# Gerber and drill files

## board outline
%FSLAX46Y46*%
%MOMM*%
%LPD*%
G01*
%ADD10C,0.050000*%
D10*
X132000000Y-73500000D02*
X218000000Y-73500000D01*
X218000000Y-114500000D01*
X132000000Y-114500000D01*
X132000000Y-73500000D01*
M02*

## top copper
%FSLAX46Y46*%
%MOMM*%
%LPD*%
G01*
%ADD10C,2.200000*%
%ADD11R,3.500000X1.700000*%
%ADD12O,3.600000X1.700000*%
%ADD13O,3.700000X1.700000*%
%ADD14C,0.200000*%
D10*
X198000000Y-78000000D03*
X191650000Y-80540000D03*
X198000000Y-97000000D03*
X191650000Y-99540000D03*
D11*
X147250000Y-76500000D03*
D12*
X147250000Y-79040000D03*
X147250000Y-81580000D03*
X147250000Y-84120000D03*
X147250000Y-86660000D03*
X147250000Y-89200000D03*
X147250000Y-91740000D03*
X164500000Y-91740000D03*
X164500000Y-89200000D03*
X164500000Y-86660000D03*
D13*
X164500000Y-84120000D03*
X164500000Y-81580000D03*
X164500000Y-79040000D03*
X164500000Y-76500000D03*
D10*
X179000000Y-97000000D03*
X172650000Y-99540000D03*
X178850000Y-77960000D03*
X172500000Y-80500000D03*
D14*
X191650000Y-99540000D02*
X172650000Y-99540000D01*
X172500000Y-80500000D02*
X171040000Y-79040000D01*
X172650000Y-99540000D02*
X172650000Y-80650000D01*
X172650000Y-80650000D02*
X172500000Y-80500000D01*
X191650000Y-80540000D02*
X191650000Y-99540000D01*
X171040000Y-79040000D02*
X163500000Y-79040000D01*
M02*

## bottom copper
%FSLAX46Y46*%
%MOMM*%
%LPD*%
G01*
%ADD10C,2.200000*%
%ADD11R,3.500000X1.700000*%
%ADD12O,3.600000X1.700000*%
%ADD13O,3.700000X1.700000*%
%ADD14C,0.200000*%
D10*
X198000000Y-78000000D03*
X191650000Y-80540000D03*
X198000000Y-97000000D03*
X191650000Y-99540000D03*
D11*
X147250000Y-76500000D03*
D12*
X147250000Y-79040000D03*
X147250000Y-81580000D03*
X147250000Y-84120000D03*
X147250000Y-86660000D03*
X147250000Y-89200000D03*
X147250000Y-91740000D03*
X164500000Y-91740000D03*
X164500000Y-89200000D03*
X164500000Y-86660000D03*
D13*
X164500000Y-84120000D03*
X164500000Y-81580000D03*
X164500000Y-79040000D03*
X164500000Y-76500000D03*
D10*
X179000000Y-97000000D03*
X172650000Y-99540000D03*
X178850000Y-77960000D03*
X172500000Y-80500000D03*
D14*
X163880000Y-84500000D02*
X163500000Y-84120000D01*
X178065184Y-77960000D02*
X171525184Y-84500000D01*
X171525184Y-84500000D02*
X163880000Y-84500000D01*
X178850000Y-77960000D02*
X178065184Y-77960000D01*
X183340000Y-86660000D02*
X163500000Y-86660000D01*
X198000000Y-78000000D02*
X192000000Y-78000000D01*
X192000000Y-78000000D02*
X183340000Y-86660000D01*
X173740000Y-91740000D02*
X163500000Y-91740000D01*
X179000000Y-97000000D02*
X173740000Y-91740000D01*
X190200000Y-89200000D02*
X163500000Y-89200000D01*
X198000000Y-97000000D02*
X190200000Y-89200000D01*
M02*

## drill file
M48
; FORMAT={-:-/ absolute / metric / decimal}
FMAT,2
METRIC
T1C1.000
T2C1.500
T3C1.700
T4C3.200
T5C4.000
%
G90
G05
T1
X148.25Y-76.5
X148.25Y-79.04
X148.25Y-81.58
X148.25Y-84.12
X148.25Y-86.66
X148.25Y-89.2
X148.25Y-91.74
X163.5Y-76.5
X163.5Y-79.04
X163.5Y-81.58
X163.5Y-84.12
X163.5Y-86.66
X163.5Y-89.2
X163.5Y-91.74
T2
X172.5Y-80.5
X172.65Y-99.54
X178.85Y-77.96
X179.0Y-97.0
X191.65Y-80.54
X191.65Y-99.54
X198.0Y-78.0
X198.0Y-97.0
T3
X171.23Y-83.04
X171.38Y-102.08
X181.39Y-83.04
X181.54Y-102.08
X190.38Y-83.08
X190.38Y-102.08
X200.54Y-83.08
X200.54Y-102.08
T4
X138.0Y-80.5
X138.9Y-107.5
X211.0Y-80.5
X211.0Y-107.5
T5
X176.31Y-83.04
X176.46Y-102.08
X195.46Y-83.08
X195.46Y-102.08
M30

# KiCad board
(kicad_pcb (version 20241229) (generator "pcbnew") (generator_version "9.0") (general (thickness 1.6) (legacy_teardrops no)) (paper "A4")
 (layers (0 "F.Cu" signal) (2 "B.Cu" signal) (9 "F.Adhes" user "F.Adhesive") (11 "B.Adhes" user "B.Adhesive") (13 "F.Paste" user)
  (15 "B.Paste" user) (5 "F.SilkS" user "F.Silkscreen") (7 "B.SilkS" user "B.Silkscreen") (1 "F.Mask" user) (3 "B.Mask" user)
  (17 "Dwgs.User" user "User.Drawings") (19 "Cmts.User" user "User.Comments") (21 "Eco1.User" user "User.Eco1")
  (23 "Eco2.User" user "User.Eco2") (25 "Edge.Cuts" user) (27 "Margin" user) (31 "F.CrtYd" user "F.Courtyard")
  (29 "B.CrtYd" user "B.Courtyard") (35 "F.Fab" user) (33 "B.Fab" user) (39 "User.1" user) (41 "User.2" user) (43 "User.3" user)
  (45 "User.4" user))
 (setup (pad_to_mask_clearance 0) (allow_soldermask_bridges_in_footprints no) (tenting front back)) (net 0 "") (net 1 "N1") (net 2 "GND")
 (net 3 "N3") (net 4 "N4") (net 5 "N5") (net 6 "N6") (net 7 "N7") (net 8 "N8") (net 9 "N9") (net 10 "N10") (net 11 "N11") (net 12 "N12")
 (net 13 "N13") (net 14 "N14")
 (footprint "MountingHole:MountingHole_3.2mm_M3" (layer "F.Cu") (at 138.9 107.5)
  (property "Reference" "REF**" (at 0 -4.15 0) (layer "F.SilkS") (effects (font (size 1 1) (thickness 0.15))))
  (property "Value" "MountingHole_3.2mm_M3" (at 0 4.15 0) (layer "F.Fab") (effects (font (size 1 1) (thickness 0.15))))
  (pad "" np_thru_hole circle (at 0 0) (size 3.2 3.2) (drill 3.2) (layers "*.Cu" "*.Mask")))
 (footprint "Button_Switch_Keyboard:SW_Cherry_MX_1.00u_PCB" (layer "F.Cu") (at 198 78)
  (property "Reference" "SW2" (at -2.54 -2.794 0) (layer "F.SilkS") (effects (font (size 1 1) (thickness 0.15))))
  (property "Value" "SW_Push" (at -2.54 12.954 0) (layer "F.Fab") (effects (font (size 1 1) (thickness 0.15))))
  (pad "" np_thru_hole circle (at -7.62 5.08) (size 1.7 1.7) (drill 1.7) (layers "*.Cu" "*.Mask"))
  (pad "" np_thru_hole circle (at -2.54 5.08) (size 4 4) (drill 4) (layers "*.Cu" "*.Mask"))
  (pad "" np_thru_hole circle (at 2.54 5.08) (size 1.7 1.7) (drill 1.7) (layers "*.Cu" "*.Mask"))
  (pad "1" thru_hole circle (at 0 0) (size 2.2 2.2) (drill 1.5) (layers "*.Cu" "*.Mask") (remove_unused_layers no) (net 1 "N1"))
  (pad "2" thru_hole circle (at -6.35 2.54) (size 2.2 2.2) (drill 1.5) (layers "*.Cu" "*.Mask") (remove_unused_layers no) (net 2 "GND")))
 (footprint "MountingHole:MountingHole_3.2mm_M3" (layer "F.Cu") (at 211 80.5)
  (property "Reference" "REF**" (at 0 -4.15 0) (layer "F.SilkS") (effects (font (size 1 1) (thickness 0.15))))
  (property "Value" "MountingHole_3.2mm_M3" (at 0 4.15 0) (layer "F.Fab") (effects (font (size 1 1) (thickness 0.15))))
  (pad "" np_thru_hole circle (at 0 0) (size 3.2 3.2) (drill 3.2) (layers "*.Cu" "*.Mask")))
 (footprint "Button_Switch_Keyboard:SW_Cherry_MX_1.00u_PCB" (layer "F.Cu") (at 198 97)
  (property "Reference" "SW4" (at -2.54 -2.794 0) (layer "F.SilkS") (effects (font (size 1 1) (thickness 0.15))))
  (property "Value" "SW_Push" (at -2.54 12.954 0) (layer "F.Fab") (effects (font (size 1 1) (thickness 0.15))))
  (pad "" np_thru_hole circle (at -7.62 5.08) (size 1.7 1.7) (drill 1.7) (layers "*.Cu" "*.Mask"))
  (pad "" np_thru_hole circle (at -2.54 5.08) (size 4 4) (drill 4) (layers "*.Cu" "*.Mask"))
  (pad "" np_thru_hole circle (at 2.54 5.08) (size 1.7 1.7) (drill 1.7) (layers "*.Cu" "*.Mask"))
  (pad "1" thru_hole circle (at 0 0) (size 2.2 2.2) (drill 1.5) (layers "*.Cu" "*.Mask") (remove_unused_layers no) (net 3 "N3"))
  (pad "2" thru_hole circle (at -6.35 2.54) (size 2.2 2.2) (drill 1.5) (layers "*.Cu" "*.Mask") (remove_unused_layers no) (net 2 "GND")))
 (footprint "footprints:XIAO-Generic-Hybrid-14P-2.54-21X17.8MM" (layer "F.Cu") (at 155.875 84.12)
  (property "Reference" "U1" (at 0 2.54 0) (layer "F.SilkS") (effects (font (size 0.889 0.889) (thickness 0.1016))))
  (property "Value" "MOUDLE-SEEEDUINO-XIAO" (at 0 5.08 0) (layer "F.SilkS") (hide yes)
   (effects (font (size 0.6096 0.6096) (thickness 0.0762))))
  (pad "1" thru_hole rect (at -7.625 -7.62) (size 3.5 1.7) (drill 1 (offset -1 0)) (layers "*.Cu" "*.Mask") (remove_unused_layers no)
   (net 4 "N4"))
  (pad "2" thru_hole oval (at -7.625 -5.08) (size 3.6 1.7) (drill 1 (offset -1 0)) (layers "*.Cu" "*.Mask") (remove_unused_layers no)
   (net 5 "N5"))
  (pad "3" thru_hole oval (at -7.625 -2.54) (size 3.6 1.7) (drill 1 (offset -1 0)) (layers "*.Cu" "*.Mask") (remove_unused_layers no)
   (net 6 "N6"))
  (pad "4" thru_hole oval (at -7.625 0) (size 3.6 1.7) (drill 1 (offset -1 0)) (layers "*.Cu" "*.Mask") (remove_unused_layers no)
   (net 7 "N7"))
  (pad "5" thru_hole oval (at -7.625 2.54) (size 3.6 1.7) (drill 1 (offset -1 0)) (layers "*.Cu" "*.Mask") (remove_unused_layers no)
   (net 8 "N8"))
  (pad "6" thru_hole oval (at -7.625 5.08 180) (size 3.6 1.7) (drill 1 (offset 1 0)) (layers "*.Cu" "*.Mask") (remove_unused_layers no)
   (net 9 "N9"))
  (pad "7" thru_hole oval (at -7.625 7.62) (size 3.6 1.7) (drill 1 (offset -1 0)) (layers "*.Cu" "*.Mask") (remove_unused_layers no)
   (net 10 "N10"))
  (pad "8" thru_hole oval (at 7.625 7.62) (size 3.6 1.7) (drill 1 (offset 1 0)) (layers "*.Cu" "*.Mask") (remove_unused_layers no)
   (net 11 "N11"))
  (pad "9" thru_hole oval (at 7.625 5.08) (size 3.6 1.7) (drill 1 (offset 1 0)) (layers "*.Cu" "*.Mask") (remove_unused_layers no)
   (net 3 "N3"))
  (pad "10" thru_hole oval (at 7.625 2.54) (size 3.6 1.7) (drill 1 (offset 1 0)) (layers "*.Cu" "*.Mask") (remove_unused_layers no)
   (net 1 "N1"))
  (pad "11" thru_hole oval (at 7.625 0) (size 3.7 1.7) (drill 1 (offset 1 0)) (layers "*.Cu" "*.Mask") (remove_unused_layers no)
   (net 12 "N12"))
  (pad "12" thru_hole oval (at 7.625 -2.54) (size 3.7 1.7) (drill 1 (offset 1 0)) (layers "*.Cu" "*.Mask") (remove_unused_layers no)
   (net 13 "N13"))
  (pad "13" thru_hole oval (at 7.625 -5.08) (size 3.7 1.7) (drill 1 (offset 1 0)) (layers "*.Cu" "*.Mask") (remove_unused_layers no)
   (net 2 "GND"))
  (pad "14" thru_hole oval (at 7.625 -7.62) (size 3.7 1.7) (drill 1 (offset 1 0)) (layers "*.Cu" "*.Mask") (remove_unused_layers no)
   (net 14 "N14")))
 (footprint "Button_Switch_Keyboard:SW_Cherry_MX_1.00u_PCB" (layer "F.Cu") (at 179 97)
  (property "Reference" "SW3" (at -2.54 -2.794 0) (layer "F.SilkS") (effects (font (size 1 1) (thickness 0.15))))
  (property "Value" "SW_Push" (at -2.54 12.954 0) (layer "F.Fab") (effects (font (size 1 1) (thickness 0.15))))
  (pad "" np_thru_hole circle (at -7.62 5.08) (size 1.7 1.7) (drill 1.7) (layers "*.Cu" "*.Mask"))
  (pad "" np_thru_hole circle (at -2.54 5.08) (size 4 4) (drill 4) (layers "*.Cu" "*.Mask"))
  (pad "" np_thru_hole circle (at 2.54 5.08) (size 1.7 1.7) (drill 1.7) (layers "*.Cu" "*.Mask"))
  (pad "1" thru_hole circle (at 0 0) (size 2.2 2.2) (drill 1.5) (layers "*.Cu" "*.Mask") (remove_unused_layers no) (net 11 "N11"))
  (pad "2" thru_hole circle (at -6.35 2.54) (size 2.2 2.2) (drill 1.5) (layers "*.Cu" "*.Mask") (remove_unused_layers no) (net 2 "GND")))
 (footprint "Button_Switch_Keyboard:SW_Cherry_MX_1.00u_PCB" (layer "F.Cu") (at 178.85 77.96)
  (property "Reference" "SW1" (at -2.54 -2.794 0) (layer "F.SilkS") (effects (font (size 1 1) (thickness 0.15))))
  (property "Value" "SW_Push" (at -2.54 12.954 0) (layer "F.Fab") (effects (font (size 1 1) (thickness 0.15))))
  (pad "" np_thru_hole circle (at -7.62 5.08) (size 1.7 1.7) (drill 1.7) (layers "*.Cu" "*.Mask"))
  (pad "" np_thru_hole circle (at -2.54 5.08) (size 4 4) (drill 4) (layers "*.Cu" "*.Mask"))
  (pad "" np_thru_hole circle (at 2.54 5.08) (size 1.7 1.7) (drill 1.7) (layers "*.Cu" "*.Mask"))
  (pad "1" thru_hole circle (at 0 0) (size 2.2 2.2) (drill 1.5) (layers "*.Cu" "*.Mask") (remove_unused_layers no) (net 12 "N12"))
  (pad "2" thru_hole circle (at -6.35 2.54) (size 2.2 2.2) (drill 1.5) (layers "*.Cu" "*.Mask") (remove_unused_layers no) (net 2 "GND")))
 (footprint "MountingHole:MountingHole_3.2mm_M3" (layer "F.Cu") (at 211 107.5)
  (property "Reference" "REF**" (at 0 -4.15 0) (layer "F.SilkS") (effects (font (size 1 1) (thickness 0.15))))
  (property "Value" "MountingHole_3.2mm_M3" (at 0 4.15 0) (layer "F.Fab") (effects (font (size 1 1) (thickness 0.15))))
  (pad "" np_thru_hole circle (at 0 0) (size 3.2 3.2) (drill 3.2) (layers "*.Cu" "*.Mask")))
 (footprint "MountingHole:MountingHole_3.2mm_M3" (layer "F.Cu") (at 138 80.5)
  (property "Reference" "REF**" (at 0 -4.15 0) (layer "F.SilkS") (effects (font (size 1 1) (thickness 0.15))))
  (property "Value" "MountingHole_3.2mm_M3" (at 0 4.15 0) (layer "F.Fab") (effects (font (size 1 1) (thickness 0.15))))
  (pad "" np_thru_hole circle (at 0 0) (size 3.2 3.2) (drill 3.2) (layers "*.Cu" "*.Mask")))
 (gr_rect (start 132 73.5) (end 218 114.5) (stroke (width 0.05) (type default)) (fill no) (layer "Edge.Cuts"))
 (segment (start 191.65 99.54) (end 172.65 99.54) (width 0.2) (layer "F.Cu") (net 2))
 (segment (start 172.5 80.5) (end 171.04 79.04) (width 0.2) (layer "F.Cu") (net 2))
 (segment (start 172.65 99.54) (end 172.65 80.65) (width 0.2) (layer "F.Cu") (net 2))
 (segment (start 172.65 80.65) (end 172.5 80.5) (width 0.2) (layer "F.Cu") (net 2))
 (segment (start 191.65 80.54) (end 191.65 99.54) (width 0.2) (layer "F.Cu") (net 2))
 (segment (start 171.04 79.04) (end 163.5 79.04) (width 0.2) (layer "F.Cu") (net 2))
 (segment (start 163.88 84.5) (end 163.5 84.12) (width 0.2) (layer "B.Cu") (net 12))
 (segment (start 178.065184 77.96) (end 171.525184 84.5) (width 0.2) (layer "B.Cu") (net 12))
 (segment (start 171.525184 84.5) (end 163.88 84.5) (width 0.2) (layer "B.Cu") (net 12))
 (segment (start 178.85 77.96) (end 178.065184 77.96) (width 0.2) (layer "B.Cu") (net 12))
 (segment (start 183.34 86.66) (end 163.5 86.66) (width 0.2) (layer "B.Cu") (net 1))
 (segment (start 198 78) (end 192 78) (width 0.2) (layer "B.Cu") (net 1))
 (segment (start 192 78) (end 183.34 86.66) (width 0.2) (layer "B.Cu") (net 1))
 (segment (start 173.74 91.74) (end 163.5 91.74) (width 0.2) (layer "B.Cu") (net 11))
 (segment (start 179 97) (end 173.74 91.74) (width 0.2) (layer "B.Cu") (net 11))
 (segment (start 190.2 89.2) (end 163.5 89.2) (width 0.2) (layer "B.Cu") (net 3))
 (segment (start 198 97) (end 190.2 89.2) (width 0.2) (layer "B.Cu") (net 3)))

